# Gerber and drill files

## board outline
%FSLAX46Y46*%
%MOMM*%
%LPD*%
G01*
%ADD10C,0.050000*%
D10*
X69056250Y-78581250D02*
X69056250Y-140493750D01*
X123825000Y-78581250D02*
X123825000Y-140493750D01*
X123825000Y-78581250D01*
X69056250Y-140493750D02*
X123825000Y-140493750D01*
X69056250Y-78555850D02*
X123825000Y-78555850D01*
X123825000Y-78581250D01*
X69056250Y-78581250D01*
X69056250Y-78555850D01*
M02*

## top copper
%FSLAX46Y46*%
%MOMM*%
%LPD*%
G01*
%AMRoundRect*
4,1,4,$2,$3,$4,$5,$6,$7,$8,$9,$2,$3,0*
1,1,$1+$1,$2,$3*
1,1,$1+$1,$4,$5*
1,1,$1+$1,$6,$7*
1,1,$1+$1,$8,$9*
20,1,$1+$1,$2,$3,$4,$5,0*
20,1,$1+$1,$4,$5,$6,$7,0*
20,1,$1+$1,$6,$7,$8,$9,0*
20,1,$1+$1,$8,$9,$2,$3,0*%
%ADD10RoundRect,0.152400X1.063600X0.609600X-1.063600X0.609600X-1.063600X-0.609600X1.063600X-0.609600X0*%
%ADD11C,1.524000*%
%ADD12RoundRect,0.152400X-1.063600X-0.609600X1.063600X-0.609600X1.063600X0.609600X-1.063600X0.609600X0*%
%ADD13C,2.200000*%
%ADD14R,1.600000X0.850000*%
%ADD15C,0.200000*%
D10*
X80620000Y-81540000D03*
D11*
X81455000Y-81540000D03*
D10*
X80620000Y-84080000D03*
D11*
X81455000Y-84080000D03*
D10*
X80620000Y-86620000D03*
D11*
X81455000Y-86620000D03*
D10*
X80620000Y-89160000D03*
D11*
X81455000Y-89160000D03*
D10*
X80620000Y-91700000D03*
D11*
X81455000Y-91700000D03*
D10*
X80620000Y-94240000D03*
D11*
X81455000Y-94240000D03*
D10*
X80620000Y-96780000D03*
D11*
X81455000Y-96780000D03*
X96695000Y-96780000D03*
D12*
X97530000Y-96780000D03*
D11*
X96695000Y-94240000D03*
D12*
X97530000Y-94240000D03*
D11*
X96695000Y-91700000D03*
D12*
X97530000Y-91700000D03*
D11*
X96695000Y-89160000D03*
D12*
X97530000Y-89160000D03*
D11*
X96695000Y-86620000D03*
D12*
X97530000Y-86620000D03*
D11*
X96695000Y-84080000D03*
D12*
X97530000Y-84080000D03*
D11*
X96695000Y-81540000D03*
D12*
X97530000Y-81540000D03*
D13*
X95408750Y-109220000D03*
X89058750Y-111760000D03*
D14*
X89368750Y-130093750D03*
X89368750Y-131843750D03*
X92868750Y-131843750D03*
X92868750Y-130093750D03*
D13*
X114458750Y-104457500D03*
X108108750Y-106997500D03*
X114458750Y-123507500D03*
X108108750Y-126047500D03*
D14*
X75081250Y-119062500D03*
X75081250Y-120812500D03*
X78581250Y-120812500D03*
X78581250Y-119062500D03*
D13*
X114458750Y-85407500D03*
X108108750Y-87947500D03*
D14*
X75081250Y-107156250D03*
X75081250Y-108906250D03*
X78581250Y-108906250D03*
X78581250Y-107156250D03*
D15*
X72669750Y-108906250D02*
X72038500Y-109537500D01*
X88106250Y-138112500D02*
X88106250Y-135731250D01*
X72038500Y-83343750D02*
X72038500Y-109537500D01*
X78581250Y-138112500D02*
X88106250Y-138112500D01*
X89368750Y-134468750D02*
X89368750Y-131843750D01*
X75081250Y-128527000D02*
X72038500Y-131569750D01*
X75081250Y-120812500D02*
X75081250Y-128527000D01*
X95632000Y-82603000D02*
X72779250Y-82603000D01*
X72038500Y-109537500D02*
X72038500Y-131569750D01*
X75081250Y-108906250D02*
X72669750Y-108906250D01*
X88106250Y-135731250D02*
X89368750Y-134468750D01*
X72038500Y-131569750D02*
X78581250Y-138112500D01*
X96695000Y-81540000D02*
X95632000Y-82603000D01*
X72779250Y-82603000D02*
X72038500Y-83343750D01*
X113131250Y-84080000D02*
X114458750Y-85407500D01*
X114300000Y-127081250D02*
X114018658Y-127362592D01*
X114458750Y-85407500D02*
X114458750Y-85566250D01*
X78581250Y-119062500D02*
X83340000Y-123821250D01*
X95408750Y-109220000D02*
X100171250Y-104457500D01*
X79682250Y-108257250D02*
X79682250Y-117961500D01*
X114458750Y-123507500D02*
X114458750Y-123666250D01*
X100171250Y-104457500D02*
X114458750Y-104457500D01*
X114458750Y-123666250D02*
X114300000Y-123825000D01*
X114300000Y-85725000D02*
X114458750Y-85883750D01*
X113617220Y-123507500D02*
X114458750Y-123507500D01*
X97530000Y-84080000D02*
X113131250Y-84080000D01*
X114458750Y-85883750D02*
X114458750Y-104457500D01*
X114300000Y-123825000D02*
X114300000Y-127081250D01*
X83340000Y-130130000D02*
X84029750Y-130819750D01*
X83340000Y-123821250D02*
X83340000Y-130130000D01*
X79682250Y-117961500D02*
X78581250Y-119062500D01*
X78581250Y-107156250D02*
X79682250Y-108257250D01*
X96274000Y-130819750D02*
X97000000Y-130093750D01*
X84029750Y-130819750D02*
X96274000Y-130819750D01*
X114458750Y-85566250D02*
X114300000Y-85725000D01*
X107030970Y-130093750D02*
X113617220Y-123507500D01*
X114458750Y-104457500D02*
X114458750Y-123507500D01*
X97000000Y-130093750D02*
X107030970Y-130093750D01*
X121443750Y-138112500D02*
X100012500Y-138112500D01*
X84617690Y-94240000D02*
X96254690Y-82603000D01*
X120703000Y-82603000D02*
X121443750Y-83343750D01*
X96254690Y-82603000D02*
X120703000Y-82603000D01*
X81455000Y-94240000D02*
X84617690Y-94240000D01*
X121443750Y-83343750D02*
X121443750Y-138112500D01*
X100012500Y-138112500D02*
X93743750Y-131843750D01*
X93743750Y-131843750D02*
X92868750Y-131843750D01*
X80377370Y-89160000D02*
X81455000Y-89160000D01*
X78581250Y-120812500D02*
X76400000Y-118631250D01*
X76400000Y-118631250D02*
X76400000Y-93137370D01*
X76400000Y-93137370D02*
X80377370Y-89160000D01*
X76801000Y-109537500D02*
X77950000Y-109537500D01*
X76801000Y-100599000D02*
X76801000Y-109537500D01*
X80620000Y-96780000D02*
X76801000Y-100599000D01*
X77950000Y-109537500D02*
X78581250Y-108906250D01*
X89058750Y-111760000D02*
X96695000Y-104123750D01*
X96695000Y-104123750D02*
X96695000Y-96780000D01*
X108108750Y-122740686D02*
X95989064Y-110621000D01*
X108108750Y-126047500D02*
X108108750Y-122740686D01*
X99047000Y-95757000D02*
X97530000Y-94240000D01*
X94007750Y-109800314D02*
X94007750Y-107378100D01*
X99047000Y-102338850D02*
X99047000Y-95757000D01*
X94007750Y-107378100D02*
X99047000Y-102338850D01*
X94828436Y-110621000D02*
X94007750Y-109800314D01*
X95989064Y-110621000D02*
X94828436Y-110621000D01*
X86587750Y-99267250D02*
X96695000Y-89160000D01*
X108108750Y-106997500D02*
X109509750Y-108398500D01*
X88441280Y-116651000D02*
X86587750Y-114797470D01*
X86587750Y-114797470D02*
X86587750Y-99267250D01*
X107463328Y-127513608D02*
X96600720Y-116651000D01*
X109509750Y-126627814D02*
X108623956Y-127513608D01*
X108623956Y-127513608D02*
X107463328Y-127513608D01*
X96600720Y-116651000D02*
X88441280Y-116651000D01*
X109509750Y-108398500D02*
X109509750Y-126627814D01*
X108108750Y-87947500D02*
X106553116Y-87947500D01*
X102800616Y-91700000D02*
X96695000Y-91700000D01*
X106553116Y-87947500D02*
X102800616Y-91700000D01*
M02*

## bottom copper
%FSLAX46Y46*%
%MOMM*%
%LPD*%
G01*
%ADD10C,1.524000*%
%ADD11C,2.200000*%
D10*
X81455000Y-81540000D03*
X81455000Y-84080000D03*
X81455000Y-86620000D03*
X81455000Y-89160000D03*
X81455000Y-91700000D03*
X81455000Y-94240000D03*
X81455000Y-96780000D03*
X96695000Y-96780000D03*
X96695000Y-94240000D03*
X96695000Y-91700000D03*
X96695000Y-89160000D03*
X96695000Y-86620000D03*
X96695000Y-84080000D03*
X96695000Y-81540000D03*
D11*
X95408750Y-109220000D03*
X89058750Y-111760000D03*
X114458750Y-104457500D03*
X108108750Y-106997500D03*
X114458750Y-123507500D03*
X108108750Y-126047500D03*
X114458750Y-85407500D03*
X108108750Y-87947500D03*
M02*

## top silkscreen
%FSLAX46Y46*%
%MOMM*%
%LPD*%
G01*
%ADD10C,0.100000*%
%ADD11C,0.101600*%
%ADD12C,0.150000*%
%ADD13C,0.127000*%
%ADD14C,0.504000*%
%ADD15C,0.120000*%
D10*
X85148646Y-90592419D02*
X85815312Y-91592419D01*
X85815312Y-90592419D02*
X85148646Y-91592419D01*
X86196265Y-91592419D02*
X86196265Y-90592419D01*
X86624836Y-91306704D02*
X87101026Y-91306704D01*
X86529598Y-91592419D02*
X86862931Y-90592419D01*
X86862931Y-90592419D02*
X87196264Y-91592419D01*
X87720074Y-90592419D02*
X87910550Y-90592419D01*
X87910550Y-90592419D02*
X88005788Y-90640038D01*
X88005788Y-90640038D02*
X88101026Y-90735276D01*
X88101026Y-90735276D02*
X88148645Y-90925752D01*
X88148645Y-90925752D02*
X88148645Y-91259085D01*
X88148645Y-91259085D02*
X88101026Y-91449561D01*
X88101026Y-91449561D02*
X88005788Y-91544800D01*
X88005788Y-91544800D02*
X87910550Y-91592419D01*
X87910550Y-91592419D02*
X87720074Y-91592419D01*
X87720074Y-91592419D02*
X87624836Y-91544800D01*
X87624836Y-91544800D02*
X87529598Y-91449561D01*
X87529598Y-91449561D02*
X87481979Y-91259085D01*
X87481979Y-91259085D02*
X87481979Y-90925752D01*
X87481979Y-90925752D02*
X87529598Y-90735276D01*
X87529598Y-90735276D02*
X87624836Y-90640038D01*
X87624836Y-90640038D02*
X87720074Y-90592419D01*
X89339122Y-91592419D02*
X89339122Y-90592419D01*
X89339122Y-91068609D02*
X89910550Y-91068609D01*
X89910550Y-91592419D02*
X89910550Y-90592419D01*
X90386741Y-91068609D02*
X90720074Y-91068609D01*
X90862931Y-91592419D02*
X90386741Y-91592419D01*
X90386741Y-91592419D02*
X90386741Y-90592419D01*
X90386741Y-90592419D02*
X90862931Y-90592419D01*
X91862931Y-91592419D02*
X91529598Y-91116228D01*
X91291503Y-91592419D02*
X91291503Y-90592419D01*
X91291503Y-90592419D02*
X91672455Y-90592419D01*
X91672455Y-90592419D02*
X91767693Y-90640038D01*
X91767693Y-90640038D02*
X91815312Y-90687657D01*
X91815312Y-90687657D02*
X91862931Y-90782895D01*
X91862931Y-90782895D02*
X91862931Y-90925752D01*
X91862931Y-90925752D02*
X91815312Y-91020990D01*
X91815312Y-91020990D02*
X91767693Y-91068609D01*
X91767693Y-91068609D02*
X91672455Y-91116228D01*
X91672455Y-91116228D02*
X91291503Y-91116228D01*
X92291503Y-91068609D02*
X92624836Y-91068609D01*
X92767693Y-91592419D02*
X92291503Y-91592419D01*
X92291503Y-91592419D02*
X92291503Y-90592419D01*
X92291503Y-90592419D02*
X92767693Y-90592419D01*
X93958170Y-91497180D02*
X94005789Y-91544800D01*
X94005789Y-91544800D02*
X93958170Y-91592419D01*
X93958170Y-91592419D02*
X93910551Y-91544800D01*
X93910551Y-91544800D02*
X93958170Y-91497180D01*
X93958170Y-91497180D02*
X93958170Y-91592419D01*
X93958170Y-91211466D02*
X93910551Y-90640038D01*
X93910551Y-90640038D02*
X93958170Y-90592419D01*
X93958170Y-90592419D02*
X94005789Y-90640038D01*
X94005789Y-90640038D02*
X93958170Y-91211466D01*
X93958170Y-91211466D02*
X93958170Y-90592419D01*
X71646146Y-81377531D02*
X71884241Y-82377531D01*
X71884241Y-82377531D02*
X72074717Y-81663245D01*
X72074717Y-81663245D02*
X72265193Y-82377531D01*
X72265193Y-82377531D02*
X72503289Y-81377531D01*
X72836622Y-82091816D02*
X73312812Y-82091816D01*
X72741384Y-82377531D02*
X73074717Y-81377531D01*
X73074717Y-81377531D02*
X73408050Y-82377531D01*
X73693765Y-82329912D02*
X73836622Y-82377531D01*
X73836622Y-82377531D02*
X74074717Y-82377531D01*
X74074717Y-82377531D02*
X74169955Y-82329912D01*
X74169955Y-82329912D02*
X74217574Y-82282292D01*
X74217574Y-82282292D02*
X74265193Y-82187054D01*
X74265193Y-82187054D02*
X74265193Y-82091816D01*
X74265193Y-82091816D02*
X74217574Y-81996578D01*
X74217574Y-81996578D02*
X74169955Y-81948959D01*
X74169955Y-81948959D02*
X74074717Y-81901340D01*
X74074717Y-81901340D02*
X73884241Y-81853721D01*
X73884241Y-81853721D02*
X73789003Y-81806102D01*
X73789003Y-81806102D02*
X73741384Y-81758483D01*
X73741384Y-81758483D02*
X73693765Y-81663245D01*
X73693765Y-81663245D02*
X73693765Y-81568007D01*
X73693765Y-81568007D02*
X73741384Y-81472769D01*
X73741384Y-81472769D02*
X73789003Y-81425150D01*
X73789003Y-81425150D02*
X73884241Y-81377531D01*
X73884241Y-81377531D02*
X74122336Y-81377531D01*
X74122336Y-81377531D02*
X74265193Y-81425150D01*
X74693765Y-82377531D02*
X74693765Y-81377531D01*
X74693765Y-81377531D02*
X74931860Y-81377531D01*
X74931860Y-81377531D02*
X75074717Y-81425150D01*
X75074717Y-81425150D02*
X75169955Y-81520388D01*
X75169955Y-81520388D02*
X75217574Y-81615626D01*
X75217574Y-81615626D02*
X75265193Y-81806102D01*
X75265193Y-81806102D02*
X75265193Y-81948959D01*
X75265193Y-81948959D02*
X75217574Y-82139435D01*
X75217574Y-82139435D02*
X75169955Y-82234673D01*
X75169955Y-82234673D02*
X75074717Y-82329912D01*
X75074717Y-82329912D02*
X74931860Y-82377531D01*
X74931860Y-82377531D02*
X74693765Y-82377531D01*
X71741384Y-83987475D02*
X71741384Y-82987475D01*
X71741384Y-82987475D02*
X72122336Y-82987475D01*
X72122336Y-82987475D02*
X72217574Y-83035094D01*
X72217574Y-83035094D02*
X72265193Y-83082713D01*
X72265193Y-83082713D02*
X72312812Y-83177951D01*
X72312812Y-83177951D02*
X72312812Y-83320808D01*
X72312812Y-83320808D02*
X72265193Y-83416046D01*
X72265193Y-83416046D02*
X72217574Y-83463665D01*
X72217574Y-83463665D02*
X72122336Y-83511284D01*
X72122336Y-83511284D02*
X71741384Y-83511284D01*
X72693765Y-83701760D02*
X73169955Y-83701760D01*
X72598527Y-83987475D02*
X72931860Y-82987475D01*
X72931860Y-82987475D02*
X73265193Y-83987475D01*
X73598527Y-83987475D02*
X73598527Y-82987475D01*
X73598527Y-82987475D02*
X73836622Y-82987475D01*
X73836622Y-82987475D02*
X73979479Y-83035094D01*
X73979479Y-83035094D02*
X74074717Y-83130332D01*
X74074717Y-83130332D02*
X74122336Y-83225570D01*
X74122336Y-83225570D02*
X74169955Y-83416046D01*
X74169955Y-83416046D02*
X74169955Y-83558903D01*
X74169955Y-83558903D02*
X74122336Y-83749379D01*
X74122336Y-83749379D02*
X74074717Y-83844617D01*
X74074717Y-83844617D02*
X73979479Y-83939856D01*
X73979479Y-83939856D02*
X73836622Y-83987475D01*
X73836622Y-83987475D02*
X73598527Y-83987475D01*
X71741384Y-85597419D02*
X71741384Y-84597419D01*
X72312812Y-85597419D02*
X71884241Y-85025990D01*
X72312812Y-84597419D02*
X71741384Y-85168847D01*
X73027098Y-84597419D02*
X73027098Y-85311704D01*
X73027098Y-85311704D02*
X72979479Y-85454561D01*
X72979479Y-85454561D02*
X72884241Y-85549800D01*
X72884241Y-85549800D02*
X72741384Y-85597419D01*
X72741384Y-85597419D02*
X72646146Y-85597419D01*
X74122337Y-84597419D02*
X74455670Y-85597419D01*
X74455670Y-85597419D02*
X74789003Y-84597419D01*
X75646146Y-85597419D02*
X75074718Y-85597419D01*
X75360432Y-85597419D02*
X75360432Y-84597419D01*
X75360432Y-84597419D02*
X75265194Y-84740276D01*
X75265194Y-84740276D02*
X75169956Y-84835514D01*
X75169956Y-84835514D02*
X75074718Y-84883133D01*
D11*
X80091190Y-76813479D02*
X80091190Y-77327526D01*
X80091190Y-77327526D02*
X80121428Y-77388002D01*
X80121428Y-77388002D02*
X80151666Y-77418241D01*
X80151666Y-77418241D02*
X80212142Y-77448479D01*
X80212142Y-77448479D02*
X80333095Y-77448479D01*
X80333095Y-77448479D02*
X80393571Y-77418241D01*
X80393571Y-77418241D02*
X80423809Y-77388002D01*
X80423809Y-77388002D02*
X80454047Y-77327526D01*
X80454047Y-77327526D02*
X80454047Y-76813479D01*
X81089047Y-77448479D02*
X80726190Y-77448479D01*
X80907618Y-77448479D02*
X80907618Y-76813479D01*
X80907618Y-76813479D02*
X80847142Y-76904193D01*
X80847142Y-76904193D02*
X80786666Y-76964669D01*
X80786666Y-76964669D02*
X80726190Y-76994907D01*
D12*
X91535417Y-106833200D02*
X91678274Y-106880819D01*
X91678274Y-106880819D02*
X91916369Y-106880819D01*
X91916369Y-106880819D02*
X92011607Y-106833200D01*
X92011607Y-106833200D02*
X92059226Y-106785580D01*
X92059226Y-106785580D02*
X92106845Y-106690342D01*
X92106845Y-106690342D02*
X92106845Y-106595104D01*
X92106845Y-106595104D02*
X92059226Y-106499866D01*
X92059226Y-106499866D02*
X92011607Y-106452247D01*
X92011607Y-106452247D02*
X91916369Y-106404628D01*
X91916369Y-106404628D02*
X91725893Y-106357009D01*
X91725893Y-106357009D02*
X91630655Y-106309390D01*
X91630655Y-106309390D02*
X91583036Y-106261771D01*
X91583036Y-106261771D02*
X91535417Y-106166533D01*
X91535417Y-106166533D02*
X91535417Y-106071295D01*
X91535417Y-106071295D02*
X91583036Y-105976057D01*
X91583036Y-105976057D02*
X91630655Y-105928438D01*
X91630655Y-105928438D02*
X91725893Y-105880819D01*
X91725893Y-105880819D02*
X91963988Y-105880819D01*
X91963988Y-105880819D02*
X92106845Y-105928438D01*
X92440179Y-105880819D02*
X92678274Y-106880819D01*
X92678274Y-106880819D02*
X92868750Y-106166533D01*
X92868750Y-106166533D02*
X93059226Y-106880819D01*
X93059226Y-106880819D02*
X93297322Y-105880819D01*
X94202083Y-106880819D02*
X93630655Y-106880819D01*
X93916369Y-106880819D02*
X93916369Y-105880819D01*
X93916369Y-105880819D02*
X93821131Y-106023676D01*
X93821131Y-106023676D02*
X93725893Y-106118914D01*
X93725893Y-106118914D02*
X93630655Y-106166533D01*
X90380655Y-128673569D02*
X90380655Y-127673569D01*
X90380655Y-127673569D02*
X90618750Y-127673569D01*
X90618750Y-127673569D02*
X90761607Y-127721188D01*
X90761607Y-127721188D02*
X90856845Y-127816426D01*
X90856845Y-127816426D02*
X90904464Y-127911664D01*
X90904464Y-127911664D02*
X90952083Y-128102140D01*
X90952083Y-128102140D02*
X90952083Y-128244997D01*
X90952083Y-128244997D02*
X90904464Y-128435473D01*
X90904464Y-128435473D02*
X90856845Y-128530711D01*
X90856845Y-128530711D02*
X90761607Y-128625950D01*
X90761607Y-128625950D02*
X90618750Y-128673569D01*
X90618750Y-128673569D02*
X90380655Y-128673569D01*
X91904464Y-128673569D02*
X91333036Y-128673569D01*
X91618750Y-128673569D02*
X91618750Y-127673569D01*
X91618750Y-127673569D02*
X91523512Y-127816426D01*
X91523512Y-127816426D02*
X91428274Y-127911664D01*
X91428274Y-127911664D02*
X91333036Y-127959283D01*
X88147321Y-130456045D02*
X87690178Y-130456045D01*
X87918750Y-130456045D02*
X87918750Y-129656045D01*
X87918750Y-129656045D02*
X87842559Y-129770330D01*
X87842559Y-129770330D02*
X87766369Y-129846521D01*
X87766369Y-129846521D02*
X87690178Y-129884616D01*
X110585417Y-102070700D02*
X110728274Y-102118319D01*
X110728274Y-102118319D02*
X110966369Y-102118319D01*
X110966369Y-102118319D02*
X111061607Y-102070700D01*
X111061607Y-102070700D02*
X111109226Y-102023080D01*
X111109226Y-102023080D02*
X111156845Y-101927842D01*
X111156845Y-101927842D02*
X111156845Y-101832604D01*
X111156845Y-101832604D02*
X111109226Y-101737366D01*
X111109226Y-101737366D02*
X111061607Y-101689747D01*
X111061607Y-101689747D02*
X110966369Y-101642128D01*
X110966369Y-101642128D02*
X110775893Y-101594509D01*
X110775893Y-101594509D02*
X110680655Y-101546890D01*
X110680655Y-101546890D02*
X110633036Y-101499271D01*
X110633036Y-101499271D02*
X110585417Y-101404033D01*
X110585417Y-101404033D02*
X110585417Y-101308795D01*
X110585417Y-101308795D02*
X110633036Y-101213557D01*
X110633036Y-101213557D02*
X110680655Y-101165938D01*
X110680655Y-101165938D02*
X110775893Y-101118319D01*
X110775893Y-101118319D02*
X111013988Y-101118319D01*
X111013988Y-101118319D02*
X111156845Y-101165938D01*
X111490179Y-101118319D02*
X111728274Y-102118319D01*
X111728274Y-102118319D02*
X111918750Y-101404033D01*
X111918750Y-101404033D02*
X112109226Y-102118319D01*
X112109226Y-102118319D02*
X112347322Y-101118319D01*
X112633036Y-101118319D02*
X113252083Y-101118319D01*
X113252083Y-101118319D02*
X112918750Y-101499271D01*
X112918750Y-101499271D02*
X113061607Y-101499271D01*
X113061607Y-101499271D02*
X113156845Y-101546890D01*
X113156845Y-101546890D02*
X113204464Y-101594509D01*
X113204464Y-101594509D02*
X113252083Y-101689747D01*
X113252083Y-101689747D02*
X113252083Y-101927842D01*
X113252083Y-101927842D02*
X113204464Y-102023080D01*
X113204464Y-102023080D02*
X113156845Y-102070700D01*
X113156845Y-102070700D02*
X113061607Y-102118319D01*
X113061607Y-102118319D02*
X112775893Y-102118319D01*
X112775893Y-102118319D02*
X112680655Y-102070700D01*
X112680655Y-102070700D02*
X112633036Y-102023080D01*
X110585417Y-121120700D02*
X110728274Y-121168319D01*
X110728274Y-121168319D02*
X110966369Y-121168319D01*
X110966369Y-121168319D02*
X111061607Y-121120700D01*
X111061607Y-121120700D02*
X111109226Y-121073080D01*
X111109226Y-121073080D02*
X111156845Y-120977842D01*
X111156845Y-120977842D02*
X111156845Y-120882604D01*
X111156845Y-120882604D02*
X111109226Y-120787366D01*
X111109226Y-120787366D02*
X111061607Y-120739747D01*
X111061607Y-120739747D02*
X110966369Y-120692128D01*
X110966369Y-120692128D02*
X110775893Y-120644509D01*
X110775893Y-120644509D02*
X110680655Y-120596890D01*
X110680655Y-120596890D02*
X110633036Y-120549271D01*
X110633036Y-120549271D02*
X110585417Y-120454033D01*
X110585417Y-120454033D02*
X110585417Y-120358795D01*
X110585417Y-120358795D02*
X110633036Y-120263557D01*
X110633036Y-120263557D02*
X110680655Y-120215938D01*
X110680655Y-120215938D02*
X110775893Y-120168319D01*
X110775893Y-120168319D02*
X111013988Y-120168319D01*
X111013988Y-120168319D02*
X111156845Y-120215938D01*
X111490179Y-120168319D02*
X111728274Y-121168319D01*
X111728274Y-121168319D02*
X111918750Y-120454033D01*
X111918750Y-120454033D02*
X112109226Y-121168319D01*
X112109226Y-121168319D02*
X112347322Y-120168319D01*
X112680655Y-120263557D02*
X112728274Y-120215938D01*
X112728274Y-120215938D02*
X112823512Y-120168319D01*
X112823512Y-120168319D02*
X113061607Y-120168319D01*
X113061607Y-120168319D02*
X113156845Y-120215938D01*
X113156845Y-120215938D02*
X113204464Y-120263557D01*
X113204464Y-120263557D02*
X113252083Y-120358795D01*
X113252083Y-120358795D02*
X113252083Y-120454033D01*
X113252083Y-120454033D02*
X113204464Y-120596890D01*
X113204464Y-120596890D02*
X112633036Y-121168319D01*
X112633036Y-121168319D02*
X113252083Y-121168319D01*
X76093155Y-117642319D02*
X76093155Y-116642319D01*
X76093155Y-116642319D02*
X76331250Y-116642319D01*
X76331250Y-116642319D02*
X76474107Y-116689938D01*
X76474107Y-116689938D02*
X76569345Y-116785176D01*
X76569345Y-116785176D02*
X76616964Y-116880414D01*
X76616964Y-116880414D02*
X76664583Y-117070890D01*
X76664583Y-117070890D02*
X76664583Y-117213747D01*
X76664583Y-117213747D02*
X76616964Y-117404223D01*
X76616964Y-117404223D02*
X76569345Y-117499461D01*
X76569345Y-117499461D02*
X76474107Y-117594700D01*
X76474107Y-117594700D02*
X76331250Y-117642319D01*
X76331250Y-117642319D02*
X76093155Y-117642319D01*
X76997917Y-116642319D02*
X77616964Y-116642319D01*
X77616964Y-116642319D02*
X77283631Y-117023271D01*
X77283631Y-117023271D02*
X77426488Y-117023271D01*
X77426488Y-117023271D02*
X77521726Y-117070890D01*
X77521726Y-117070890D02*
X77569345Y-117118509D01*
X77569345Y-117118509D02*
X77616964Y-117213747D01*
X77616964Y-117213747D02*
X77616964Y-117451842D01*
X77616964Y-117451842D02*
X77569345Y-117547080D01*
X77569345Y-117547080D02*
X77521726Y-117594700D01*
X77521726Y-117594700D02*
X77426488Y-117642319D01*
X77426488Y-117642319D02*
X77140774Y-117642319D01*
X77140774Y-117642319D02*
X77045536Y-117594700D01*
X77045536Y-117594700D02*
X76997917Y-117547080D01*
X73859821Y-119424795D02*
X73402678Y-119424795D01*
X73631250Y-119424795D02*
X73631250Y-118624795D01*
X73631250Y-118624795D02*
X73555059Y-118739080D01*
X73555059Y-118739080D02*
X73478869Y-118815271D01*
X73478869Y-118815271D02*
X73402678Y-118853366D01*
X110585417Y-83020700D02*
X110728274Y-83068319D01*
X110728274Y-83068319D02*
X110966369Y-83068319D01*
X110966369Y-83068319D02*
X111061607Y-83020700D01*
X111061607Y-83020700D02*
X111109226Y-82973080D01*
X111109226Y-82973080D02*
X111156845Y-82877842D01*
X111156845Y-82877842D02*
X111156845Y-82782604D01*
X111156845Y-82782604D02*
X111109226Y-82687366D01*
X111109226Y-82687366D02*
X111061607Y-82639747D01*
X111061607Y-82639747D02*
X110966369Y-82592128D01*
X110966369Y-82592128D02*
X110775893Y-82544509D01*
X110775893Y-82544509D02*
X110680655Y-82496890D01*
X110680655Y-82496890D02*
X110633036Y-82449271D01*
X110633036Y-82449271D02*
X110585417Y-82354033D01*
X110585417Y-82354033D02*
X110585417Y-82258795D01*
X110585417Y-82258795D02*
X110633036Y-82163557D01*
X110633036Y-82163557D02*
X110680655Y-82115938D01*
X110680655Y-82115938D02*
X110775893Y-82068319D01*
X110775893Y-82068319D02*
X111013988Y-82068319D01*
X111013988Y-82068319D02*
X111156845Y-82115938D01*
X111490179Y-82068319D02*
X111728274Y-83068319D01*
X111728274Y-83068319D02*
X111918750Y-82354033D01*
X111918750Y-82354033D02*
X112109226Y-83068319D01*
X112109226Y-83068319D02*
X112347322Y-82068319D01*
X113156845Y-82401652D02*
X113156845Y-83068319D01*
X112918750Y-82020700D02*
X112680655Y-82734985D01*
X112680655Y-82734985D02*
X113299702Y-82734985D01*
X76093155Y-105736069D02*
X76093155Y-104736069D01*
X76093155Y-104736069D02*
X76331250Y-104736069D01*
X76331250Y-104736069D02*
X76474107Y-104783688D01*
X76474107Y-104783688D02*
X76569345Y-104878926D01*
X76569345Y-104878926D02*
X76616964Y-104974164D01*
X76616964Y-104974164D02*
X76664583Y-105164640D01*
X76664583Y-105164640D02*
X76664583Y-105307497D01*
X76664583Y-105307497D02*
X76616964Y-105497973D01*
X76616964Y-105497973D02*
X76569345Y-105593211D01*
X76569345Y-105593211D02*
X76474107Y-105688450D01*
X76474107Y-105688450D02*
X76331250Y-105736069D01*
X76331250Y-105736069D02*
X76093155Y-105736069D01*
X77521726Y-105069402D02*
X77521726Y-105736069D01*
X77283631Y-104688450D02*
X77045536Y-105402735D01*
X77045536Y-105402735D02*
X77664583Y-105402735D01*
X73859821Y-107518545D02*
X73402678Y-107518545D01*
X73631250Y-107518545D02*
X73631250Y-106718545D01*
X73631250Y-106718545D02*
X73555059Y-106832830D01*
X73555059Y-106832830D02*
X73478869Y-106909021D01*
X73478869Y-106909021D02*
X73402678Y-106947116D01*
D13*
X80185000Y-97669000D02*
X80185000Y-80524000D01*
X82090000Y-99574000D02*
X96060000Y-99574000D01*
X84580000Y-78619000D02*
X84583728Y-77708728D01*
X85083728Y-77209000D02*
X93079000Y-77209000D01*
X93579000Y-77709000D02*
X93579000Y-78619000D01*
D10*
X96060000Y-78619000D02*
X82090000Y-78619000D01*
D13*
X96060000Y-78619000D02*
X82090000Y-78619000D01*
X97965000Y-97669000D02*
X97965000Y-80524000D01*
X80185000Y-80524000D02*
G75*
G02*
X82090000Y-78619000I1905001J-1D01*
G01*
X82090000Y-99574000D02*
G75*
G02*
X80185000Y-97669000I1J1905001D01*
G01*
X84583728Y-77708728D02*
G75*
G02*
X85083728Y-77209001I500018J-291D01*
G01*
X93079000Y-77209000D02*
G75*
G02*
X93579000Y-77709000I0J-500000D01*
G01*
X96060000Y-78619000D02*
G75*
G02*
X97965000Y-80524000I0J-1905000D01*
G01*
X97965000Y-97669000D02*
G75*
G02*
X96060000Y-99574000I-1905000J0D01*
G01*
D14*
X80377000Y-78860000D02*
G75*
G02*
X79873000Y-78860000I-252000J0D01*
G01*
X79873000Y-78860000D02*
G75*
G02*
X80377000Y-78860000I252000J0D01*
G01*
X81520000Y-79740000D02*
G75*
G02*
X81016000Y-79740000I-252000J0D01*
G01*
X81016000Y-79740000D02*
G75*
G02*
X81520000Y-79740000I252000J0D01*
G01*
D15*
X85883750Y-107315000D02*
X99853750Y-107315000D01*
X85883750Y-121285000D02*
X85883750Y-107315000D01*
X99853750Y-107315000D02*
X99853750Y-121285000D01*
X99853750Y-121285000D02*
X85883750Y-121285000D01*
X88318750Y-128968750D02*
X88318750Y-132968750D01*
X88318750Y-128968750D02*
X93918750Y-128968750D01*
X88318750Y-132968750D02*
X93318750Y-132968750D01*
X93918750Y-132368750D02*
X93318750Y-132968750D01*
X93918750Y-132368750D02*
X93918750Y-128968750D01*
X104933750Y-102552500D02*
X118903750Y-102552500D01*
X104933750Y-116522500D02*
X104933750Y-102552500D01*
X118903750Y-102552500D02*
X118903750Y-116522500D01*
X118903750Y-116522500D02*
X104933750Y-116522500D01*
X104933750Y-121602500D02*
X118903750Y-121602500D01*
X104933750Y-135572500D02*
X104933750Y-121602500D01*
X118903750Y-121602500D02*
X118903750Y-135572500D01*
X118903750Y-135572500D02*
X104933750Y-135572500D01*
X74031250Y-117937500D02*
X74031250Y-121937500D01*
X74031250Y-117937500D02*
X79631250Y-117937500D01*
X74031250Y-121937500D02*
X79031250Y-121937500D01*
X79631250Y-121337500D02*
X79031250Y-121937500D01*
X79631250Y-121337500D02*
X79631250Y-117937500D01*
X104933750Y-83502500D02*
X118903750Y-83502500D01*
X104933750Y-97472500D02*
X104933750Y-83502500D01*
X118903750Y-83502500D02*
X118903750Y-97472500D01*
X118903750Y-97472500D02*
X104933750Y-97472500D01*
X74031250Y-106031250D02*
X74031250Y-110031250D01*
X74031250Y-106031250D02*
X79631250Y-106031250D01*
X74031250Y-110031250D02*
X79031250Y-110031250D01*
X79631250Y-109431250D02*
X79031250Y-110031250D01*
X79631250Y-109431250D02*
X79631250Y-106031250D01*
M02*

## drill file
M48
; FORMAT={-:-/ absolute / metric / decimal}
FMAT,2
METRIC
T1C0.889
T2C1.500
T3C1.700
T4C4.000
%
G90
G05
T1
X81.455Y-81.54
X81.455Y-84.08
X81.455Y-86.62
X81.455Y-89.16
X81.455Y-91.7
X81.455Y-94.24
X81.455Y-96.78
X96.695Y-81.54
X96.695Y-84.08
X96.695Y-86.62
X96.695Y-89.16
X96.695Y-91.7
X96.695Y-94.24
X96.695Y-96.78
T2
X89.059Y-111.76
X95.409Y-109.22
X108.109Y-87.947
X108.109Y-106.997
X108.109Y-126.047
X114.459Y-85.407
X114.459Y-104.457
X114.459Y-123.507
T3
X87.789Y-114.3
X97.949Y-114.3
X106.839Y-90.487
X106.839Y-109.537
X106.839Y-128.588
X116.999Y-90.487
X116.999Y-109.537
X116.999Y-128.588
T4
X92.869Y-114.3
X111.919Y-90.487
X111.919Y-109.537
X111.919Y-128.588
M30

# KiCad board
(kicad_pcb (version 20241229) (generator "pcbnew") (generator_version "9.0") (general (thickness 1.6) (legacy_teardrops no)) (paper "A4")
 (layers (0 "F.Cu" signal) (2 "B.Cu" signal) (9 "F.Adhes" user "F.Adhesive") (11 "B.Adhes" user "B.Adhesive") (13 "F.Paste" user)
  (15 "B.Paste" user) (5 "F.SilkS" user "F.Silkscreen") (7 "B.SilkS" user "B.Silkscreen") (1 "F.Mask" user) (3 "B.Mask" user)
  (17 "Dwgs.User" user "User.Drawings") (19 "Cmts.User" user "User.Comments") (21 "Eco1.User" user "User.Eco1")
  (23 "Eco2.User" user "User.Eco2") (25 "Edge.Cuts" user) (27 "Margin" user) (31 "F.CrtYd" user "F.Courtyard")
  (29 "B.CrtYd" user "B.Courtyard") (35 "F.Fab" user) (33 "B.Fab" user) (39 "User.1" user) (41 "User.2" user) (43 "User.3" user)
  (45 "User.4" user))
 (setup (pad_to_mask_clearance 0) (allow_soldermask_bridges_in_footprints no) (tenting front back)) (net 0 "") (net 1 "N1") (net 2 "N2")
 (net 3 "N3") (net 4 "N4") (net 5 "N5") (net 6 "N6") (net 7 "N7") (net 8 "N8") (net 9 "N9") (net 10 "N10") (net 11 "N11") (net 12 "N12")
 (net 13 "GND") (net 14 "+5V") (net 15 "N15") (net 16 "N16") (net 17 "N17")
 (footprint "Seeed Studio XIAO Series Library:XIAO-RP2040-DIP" (layer "F.Cu") (at 89.075 89.16)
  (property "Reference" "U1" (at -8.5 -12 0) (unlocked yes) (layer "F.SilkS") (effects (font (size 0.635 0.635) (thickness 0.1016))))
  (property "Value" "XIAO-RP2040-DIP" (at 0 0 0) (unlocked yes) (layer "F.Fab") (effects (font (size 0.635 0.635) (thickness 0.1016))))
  (fp_line (start -8.89 8.509) (end -8.89 -8.636) (stroke (width 0.127) (type solid)) (layer "F.SilkS"))
  (fp_line (start -6.985 10.414) (end 6.985 10.414) (stroke (width 0.127) (type solid)) (layer "F.SilkS"))
  (fp_line (start -4.495 -10.541) (end -4.491272 -11.451272) (stroke (width 0.127) (type solid)) (layer "F.SilkS"))
  (fp_line (start -3.991272 -11.951) (end 4.004 -11.951) (stroke (width 0.127) (type solid)) (layer "F.SilkS"))
  (fp_line (start 4.504 -11.451) (end 4.504 -10.541) (stroke (width 0.127) (type solid)) (layer "F.SilkS"))
  (fp_line (start 6.985 -10.541) (end -6.985 -10.541) (stroke (width 0.1) (type solid)) (layer "F.SilkS"))
  (fp_line (start 6.985 -10.541) (end -6.985 -10.541) (stroke (width 0.127) (type solid)) (layer "F.SilkS"))
  (fp_line (start 8.89 8.509) (end 8.89 -8.636) (stroke (width 0.127) (type solid)) (layer "F.SilkS"))
  (fp_arc (start -8.89 -8.636) (mid -8.332038 -9.983038) (end -6.985 -10.541) (stroke (width 0.127) (type solid)) (layer "F.SilkS"))
  (fp_arc (start -6.985 10.414) (mid -8.332038 9.856038) (end -8.89 8.509) (stroke (width 0.127) (type solid)) (layer "F.SilkS"))
  (fp_arc (start -4.491272 -11.451272) (mid -4.344728 -11.80464) (end -3.991272 -11.951) (stroke (width 0.127) (type default))
   (layer "F.SilkS"))
  (fp_arc (start 4.004 -11.951) (mid 4.357553 -11.804553) (end 4.504 -11.451) (stroke (width 0.127) (type default)) (layer "F.SilkS"))
  (fp_arc (start 6.985 -10.541) (mid 8.332038 -9.983038) (end 8.89 -8.636) (stroke (width 0.127) (type solid)) (layer "F.SilkS"))
  (fp_arc (start 8.89 8.509) (mid 8.332038 9.856038) (end 6.985 10.414) (stroke (width 0.127) (type solid)) (layer "F.SilkS"))
  (fp_circle (center -8.95 -10.3) (end -8.95 -10.554) (stroke (width 0.5) (type solid)) (fill yes) (layer "F.SilkS"))
  (fp_circle (center -7.807 -9.42) (end -7.807 -9.674) (stroke (width 0.5) (type solid)) (fill yes) (layer "F.SilkS"))
  (pad "1" smd roundrect (at -8.455 -7.62 180) (size 2.432 1.524) (layers "F.Cu" "F.Mask") (roundrect_rratio 0.1) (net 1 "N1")
   (thermal_bridge_angle 45))
  (pad "1" thru_hole circle (at -7.62 -7.62 180) (size 1.524 1.524) (drill 0.889) (layers "*.Cu" "*.Mask") (remove_unused_layers no)
   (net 1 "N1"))
  (pad "2" smd roundrect (at -8.455 -5.08 180) (size 2.432 1.524) (layers "F.Cu" "F.Mask") (roundrect_rratio 0.1) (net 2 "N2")
   (thermal_bridge_angle 45))
  (pad "2" thru_hole circle (at -7.62 -5.08 180) (size 1.524 1.524) (drill 0.889) (layers "*.Cu" "*.Mask") (remove_unused_layers no)
   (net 2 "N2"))
  (pad "3" smd roundrect (at -8.455 -2.54 180) (size 2.432 1.524) (layers "F.Cu" "F.Mask") (roundrect_rratio 0.1) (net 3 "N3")
   (thermal_bridge_angle 45))
  (pad "3" thru_hole circle (at -7.62 -2.54 180) (size 1.524 1.524) (drill 0.889) (layers "*.Cu" "*.Mask") (remove_unused_layers no)
   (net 3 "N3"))
  (pad "4" smd roundrect (at -8.455 0 180) (size 2.432 1.524) (layers "F.Cu" "F.Mask") (roundrect_rratio 0.1) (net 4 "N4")
   (thermal_bridge_angle 45))
  (pad "4" thru_hole circle (at -7.62 0 180) (size 1.524 1.524) (drill 0.889) (layers "*.Cu" "*.Mask") (remove_unused_layers no)
   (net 4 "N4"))
  (pad "5" smd roundrect (at -8.455 2.54 180) (size 2.432 1.524) (layers "F.Cu" "F.Mask") (roundrect_rratio 0.1) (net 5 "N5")
   (thermal_bridge_angle 45))
  (pad "5" thru_hole circle (at -7.62 2.54 180) (size 1.524 1.524) (drill 0.889) (layers "*.Cu" "*.Mask") (remove_unused_layers no)
   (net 5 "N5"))
  (pad "6" smd roundrect (at -8.455 5.08 180) (size 2.432 1.524) (layers "F.Cu" "F.Mask") (roundrect_rratio 0.1) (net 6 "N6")
   (thermal_bridge_angle 45))
  (pad "6" thru_hole circle (at -7.62 5.08 180) (size 1.524 1.524) (drill 0.889) (layers "*.Cu" "*.Mask") (remove_unused_layers no)
   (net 6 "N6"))
  (pad "7" smd roundrect (at -8.455 7.62 180) (size 2.432 1.524) (layers "F.Cu" "F.Mask") (roundrect_rratio 0.1) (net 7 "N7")
   (thermal_bridge_angle 45))
  (pad "7" thru_hole circle (at -7.62 7.62 180) (size 1.524 1.524) (drill 0.889) (layers "*.Cu" "*.Mask") (remove_unused_layers no)
   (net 7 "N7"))
  (pad "8" thru_hole circle (at 7.62 7.62) (size 1.524 1.524) (drill 0.889) (layers "*.Cu" "*.Mask") (remove_unused_layers no) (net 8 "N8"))
  (pad "8" smd roundrect (at 8.455 7.62) (size 2.432 1.524) (layers "F.Cu" "F.Mask") (roundrect_rratio 0.1) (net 8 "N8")
   (thermal_bridge_angle 45))
  (pad "9" thru_hole circle (at 7.62 5.08) (size 1.524 1.524) (drill 0.889) (layers "*.Cu" "*.Mask") (remove_unused_layers no) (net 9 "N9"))
  (pad "9" smd roundrect (at 8.455 5.08) (size 2.432 1.524) (layers "F.Cu" "F.Mask") (roundrect_rratio 0.1) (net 9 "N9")
   (thermal_bridge_angle 45))
  (pad "10" thru_hole circle (at 7.62 2.54) (size 1.524 1.524) (drill 0.889) (layers "*.Cu" "*.Mask") (remove_unused_layers no)
   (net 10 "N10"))
  (pad "10" smd roundrect (at 8.455 2.54) (size 2.432 1.524) (layers "F.Cu" "F.Mask") (roundrect_rratio 0.1) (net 10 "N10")
   (thermal_bridge_angle 45))
  (pad "11" thru_hole circle (at 7.62 0) (size 1.524 1.524) (drill 0.889) (layers "*.Cu" "*.Mask") (remove_unused_layers no) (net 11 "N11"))
  (pad "11" smd roundrect (at 8.455 0) (size 2.432 1.524) (layers "F.Cu" "F.Mask") (roundrect_rratio 0.1) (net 11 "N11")
   (thermal_bridge_angle 45))
  (pad "12" thru_hole circle (at 7.62 -2.54) (size 1.524 1.524) (drill 0.889) (layers "*.Cu" "*.Mask") (remove_unused_layers no)
   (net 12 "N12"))
  (pad "12" smd roundrect (at 8.455 -2.54) (size 2.432 1.524) (layers "F.Cu" "F.Mask") (roundrect_rratio 0.1) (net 12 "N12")
   (thermal_bridge_angle 45))
  (pad "13" thru_hole circle (at 7.62 -5.08) (size 1.524 1.524) (drill 0.889) (layers "*.Cu" "*.Mask") (remove_unused_layers no)
   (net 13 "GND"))
  (pad "13" smd roundrect (at 8.455 -5.08) (size 2.432 1.524) (layers "F.Cu" "F.Mask") (roundrect_rratio 0.1) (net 13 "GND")
   (thermal_bridge_angle 45))
  (pad "14" thru_hole circle (at 7.62 -7.62) (size 1.524 1.524) (drill 0.889) (layers "*.Cu" "*.Mask") (remove_unused_layers no)
   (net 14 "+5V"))
  (pad "14" smd roundrect (at 8.455 -7.62) (size 2.432 1.524) (layers "F.Cu" "F.Mask") (roundrect_rratio 0.1) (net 14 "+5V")
   (thermal_bridge_angle 45)))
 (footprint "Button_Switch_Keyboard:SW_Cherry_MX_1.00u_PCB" (layer "F.Cu") (at 95.40875 109.22)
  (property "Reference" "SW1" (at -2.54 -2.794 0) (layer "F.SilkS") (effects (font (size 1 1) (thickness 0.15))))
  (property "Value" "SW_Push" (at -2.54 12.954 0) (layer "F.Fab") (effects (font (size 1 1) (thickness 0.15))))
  (fp_line (start -9.525 -1.905) (end 4.445 -1.905) (stroke (width 0.12) (type solid)) (layer "F.SilkS"))
  (fp_line (start -9.525 12.065) (end -9.525 -1.905) (stroke (width 0.12) (type solid)) (layer "F.SilkS"))
  (fp_line (start 4.445 -1.905) (end 4.445 12.065) (stroke (width 0.12) (type solid)) (layer "F.SilkS"))
  (fp_line (start 4.445 12.065) (end -9.525 12.065) (stroke (width 0.12) (type solid)) (layer "F.SilkS"))
  (pad "" np_thru_hole circle (at -7.62 5.08) (size 1.7 1.7) (drill 1.7) (layers "*.Cu" "*.Mask"))
  (pad "" np_thru_hole circle (at -2.54 5.08) (size 4 4) (drill 4) (layers "*.Cu" "*.Mask"))
  (pad "" np_thru_hole circle (at 2.54 5.08) (size 1.7 1.7) (drill 1.7) (layers "*.Cu" "*.Mask"))
  (pad "1" thru_hole circle (at 0 0) (size 2.2 2.2) (drill 1.5) (layers "*.Cu" "*.Mask") (remove_unused_layers no) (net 13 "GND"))
  (pad "2" thru_hole circle (at -6.35 2.54) (size 2.2 2.2) (drill 1.5) (layers "*.Cu" "*.Mask") (remove_unused_layers no) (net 8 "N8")))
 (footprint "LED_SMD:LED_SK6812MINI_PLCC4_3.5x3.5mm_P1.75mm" (layer "F.Cu") (at 91.11875 130.96875)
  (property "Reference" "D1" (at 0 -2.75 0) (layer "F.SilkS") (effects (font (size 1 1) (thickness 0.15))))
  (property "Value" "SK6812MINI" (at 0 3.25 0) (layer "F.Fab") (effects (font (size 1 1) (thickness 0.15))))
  (fp_line (start -2.8 -2) (end -2.8 2) (stroke (width 0.12) (type default)) (layer "F.SilkS"))
  (fp_line (start -2.8 -2) (end 2.8 -2) (stroke (width 0.12) (type solid)) (layer "F.SilkS"))
  (fp_line (start -2.8 2) (end 2.2 2) (stroke (width 0.12) (type solid)) (layer "F.SilkS"))
  (fp_line (start 2.8 1.4) (end 2.2 2) (stroke (width 0.12) (type default)) (layer "F.SilkS"))
  (fp_line (start 2.8 1.4) (end 2.8 -2) (stroke (width 0.12) (type solid)) (layer "F.SilkS"))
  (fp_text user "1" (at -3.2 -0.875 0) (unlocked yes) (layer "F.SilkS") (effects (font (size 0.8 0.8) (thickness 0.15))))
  (pad "1" smd rect (at -1.75 -0.875) (size 1.6 0.85) (layers "F.Cu" "F.Mask" "F.Paste") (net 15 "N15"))
  (pad "2" smd rect (at -1.75 0.875) (size 1.6 0.85) (layers "F.Cu" "F.Mask" "F.Paste") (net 14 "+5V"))
  (pad "3" smd rect (at 1.75 0.875) (size 1.6 0.85) (layers "F.Cu" "F.Mask" "F.Paste") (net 6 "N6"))
  (pad "4" smd rect (at 1.75 -0.875) (size 1.6 0.85) (layers "F.Cu" "F.Mask" "F.Paste") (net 13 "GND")))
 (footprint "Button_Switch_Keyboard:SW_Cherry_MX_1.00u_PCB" (layer "F.Cu") (at 114.45875 104.4575)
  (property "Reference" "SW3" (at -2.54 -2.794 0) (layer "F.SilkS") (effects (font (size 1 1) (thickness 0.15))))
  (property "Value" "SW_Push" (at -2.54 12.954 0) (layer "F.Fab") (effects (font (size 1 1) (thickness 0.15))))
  (fp_line (start -9.525 -1.905) (end 4.445 -1.905) (stroke (width 0.12) (type solid)) (layer "F.SilkS"))
  (fp_line (start -9.525 12.065) (end -9.525 -1.905) (stroke (width 0.12) (type solid)) (layer "F.SilkS"))
  (fp_line (start 4.445 -1.905) (end 4.445 12.065) (stroke (width 0.12) (type solid)) (layer "F.SilkS"))
  (fp_line (start 4.445 12.065) (end -9.525 12.065) (stroke (width 0.12) (type solid)) (layer "F.SilkS"))
  (pad "" np_thru_hole circle (at -7.62 5.08) (size 1.7 1.7) (drill 1.7) (layers "*.Cu" "*.Mask"))
  (pad "" np_thru_hole circle (at -2.54 5.08) (size 4 4) (drill 4) (layers "*.Cu" "*.Mask"))
  (pad "" np_thru_hole circle (at 2.54 5.08) (size 1.7 1.7) (drill 1.7) (layers "*.Cu" "*.Mask"))
  (pad "1" thru_hole circle (at 0 0) (size 2.2 2.2) (drill 1.5) (layers "*.Cu" "*.Mask") (remove_unused_layers no) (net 13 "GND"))
  (pad "2" thru_hole circle (at -6.35 2.54) (size 2.2 2.2) (drill 1.5) (layers "*.Cu" "*.Mask") (remove_unused_layers no) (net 11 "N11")))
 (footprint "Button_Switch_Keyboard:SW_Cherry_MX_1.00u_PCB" (layer "F.Cu") (at 114.45875 123.5075)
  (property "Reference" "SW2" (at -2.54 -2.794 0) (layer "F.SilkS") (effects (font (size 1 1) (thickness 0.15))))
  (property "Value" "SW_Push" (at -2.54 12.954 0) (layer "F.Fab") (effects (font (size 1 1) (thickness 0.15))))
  (fp_line (start -9.525 -1.905) (end 4.445 -1.905) (stroke (width 0.12) (type solid)) (layer "F.SilkS"))
  (fp_line (start -9.525 12.065) (end -9.525 -1.905) (stroke (width 0.12) (type solid)) (layer "F.SilkS"))
  (fp_line (start 4.445 -1.905) (end 4.445 12.065) (stroke (width 0.12) (type solid)) (layer "F.SilkS"))
  (fp_line (start 4.445 12.065) (end -9.525 12.065) (stroke (width 0.12) (type solid)) (layer "F.SilkS"))
  (pad "" np_thru_hole circle (at -7.62 5.08) (size 1.7 1.7) (drill 1.7) (layers "*.Cu" "*.Mask"))
  (pad "" np_thru_hole circle (at -2.54 5.08) (size 4 4) (drill 4) (layers "*.Cu" "*.Mask"))
  (pad "" np_thru_hole circle (at 2.54 5.08) (size 1.7 1.7) (drill 1.7) (layers "*.Cu" "*.Mask"))
  (pad "1" thru_hole circle (at 0 0) (size 2.2 2.2) (drill 1.5) (layers "*.Cu" "*.Mask") (remove_unused_layers no) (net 13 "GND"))
  (pad "2" thru_hole circle (at -6.35 2.54) (size 2.2 2.2) (drill 1.5) (layers "*.Cu" "*.Mask") (remove_unused_layers no) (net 9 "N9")))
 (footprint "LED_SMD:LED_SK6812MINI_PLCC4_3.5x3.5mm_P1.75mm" (layer "F.Cu") (at 76.83125 119.9375)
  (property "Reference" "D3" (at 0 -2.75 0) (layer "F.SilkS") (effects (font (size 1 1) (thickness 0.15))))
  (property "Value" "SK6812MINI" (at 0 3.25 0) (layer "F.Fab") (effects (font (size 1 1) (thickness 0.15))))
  (fp_line (start -2.8 -2) (end -2.8 2) (stroke (width 0.12) (type default)) (layer "F.SilkS"))
  (fp_line (start -2.8 -2) (end 2.8 -2) (stroke (width 0.12) (type solid)) (layer "F.SilkS"))
  (fp_line (start -2.8 2) (end 2.2 2) (stroke (width 0.12) (type solid)) (layer "F.SilkS"))
  (fp_line (start 2.8 1.4) (end 2.2 2) (stroke (width 0.12) (type default)) (layer "F.SilkS"))
  (fp_line (start 2.8 1.4) (end 2.8 -2) (stroke (width 0.12) (type solid)) (layer "F.SilkS"))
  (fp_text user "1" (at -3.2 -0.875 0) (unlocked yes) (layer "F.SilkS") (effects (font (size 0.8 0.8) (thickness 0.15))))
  (pad "1" smd rect (at -1.75 -0.875) (size 1.6 0.85) (layers "F.Cu" "F.Mask" "F.Paste") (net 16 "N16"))
  (pad "2" smd rect (at -1.75 0.875) (size 1.6 0.85) (layers "F.Cu" "F.Mask" "F.Paste") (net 14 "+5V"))
  (pad "3" smd rect (at 1.75 0.875) (size 1.6 0.85) (layers "F.Cu" "F.Mask" "F.Paste") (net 4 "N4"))
  (pad "4" smd rect (at 1.75 -0.875) (size 1.6 0.85) (layers "F.Cu" "F.Mask" "F.Paste") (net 13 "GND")))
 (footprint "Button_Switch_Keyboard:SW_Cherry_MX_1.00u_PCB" (layer "F.Cu") (at 114.45875 85.4075)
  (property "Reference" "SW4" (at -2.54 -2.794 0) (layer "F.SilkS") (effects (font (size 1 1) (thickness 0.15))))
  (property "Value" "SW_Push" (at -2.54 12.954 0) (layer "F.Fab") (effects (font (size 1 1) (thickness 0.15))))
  (fp_line (start -9.525 -1.905) (end 4.445 -1.905) (stroke (width 0.12) (type solid)) (layer "F.SilkS"))
  (fp_line (start -9.525 12.065) (end -9.525 -1.905) (stroke (width 0.12) (type solid)) (layer "F.SilkS"))
  (fp_line (start 4.445 -1.905) (end 4.445 12.065) (stroke (width 0.12) (type solid)) (layer "F.SilkS"))
  (fp_line (start 4.445 12.065) (end -9.525 12.065) (stroke (width 0.12) (type solid)) (layer "F.SilkS"))
  (pad "" np_thru_hole circle (at -7.62 5.08) (size 1.7 1.7) (drill 1.7) (layers "*.Cu" "*.Mask"))
  (pad "" np_thru_hole circle (at -2.54 5.08) (size 4 4) (drill 4) (layers "*.Cu" "*.Mask"))
  (pad "" np_thru_hole circle (at 2.54 5.08) (size 1.7 1.7) (drill 1.7) (layers "*.Cu" "*.Mask"))
  (pad "1" thru_hole circle (at 0 0) (size 2.2 2.2) (drill 1.5) (layers "*.Cu" "*.Mask") (remove_unused_layers no) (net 13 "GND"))
  (pad "2" thru_hole circle (at -6.35 2.54) (size 2.2 2.2) (drill 1.5) (layers "*.Cu" "*.Mask") (remove_unused_layers no) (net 10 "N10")))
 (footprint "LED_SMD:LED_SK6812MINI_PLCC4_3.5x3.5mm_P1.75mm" (layer "F.Cu") (at 76.83125 108.03125)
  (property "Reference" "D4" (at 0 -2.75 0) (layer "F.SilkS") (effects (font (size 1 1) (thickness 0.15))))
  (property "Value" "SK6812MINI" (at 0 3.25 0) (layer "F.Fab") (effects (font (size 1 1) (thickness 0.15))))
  (fp_line (start -2.8 -2) (end -2.8 2) (stroke (width 0.12) (type default)) (layer "F.SilkS"))
  (fp_line (start -2.8 -2) (end 2.8 -2) (stroke (width 0.12) (type solid)) (layer "F.SilkS"))
  (fp_line (start -2.8 2) (end 2.2 2) (stroke (width 0.12) (type solid)) (layer "F.SilkS"))
  (fp_line (start 2.8 1.4) (end 2.2 2) (stroke (width 0.12) (type default)) (layer "F.SilkS"))
  (fp_line (start 2.8 1.4) (end 2.8 -2) (stroke (width 0.12) (type solid)) (layer "F.SilkS"))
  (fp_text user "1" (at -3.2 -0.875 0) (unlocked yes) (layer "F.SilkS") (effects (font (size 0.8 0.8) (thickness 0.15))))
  (pad "1" smd rect (at -1.75 -0.875) (size 1.6 0.85) (layers "F.Cu" "F.Mask" "F.Paste") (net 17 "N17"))
  (pad "2" smd rect (at -1.75 0.875) (size 1.6 0.85) (layers "F.Cu" "F.Mask" "F.Paste") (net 14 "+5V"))
  (pad "3" smd rect (at 1.75 0.875) (size 1.6 0.85) (layers "F.Cu" "F.Mask" "F.Paste") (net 7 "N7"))
  (pad "4" smd rect (at 1.75 -0.875) (size 1.6 0.85) (layers "F.Cu" "F.Mask" "F.Paste") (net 13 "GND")))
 (gr_line (start 69.05625 78.58125) (end 69.05625 140.49375) (stroke (width 0.05) (type default)) (layer "Edge.Cuts"))
 (gr_rect (start 123.825 78.58125) (end 123.825 140.49375) (stroke (width 0.05) (type default)) (fill no) (layer "Edge.Cuts"))
 (gr_line (start 69.05625 140.49375) (end 123.825 140.49375) (stroke (width 0.05) (type default)) (layer "Edge.Cuts"))
 (gr_rect (start 69.05625 78.55585) (end 123.825 78.58125) (stroke (width 0.05) (type default)) (fill no) (layer "Edge.Cuts"))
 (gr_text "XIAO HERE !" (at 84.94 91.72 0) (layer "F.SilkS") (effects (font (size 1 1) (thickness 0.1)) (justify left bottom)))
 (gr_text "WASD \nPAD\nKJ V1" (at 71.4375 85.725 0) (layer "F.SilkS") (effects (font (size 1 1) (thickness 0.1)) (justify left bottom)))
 (segment (start 72.66975 108.90625) (end 72.0385 109.5375) (width 0.2) (layer "F.Cu") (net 14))
 (segment (start 88.10625 138.1125) (end 88.10625 135.73125) (width 0.2) (layer "F.Cu") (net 14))
 (segment (start 72.0385 83.34375) (end 72.0385 109.5375) (width 0.2) (layer "F.Cu") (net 14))
 (segment (start 78.58125 138.1125) (end 88.10625 138.1125) (width 0.2) (layer "F.Cu") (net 14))
 (segment (start 89.36875 134.46875) (end 89.36875 131.84375) (width 0.2) (layer "F.Cu") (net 14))
 (segment (start 75.08125 128.527) (end 72.0385 131.56975) (width 0.2) (layer "F.Cu") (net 14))
 (segment (start 75.08125 120.8125) (end 75.08125 128.527) (width 0.2) (layer "F.Cu") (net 14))
 (segment (start 95.632 82.603) (end 72.77925 82.603) (width 0.2) (layer "F.Cu") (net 14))
 (segment (start 72.0385 109.5375) (end 72.0385 131.56975) (width 0.2) (layer "F.Cu") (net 14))
 (segment (start 75.08125 108.90625) (end 72.66975 108.90625) (width 0.2) (layer "F.Cu") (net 14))
 (segment (start 88.10625 135.73125) (end 89.36875 134.46875) (width 0.2) (layer "F.Cu") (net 14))
 (segment (start 72.0385 131.56975) (end 78.58125 138.1125) (width 0.2) (layer "F.Cu") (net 14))
 (segment (start 96.695 81.54) (end 95.632 82.603) (width 0.2) (layer "F.Cu") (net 14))
 (segment (start 72.77925 82.603) (end 72.0385 83.34375) (width 0.2) (layer "F.Cu") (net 14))
 (segment (start 113.13125 84.08) (end 114.45875 85.4075) (width 0.2) (layer "F.Cu") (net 13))
 (segment (start 114.3 127.08125) (end 114.018658 127.362592) (width 0.2) (layer "F.Cu") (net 13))
 (segment (start 114.45875 85.4075) (end 114.45875 85.56625) (width 0.2) (layer "F.Cu") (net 13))
 (segment (start 78.58125 119.0625) (end 83.34 123.82125) (width 0.2) (layer "F.Cu") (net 13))
 (segment (start 95.40875 109.22) (end 100.17125 104.4575) (width 0.2) (layer "F.Cu") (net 13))
 (segment (start 79.68225 108.25725) (end 79.68225 117.9615) (width 0.2) (layer "F.Cu") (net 13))
 (segment (start 114.45875 123.5075) (end 114.45875 123.66625) (width 0.2) (layer "F.Cu") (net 13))
 (segment (start 100.17125 104.4575) (end 114.45875 104.4575) (width 0.2) (layer "F.Cu") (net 13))
 (segment (start 114.45875 123.66625) (end 114.3 123.825) (width 0.2) (layer "F.Cu") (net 13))
 (segment (start 114.3 85.725) (end 114.45875 85.88375) (width 0.2) (layer "F.Cu") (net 13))
 (segment (start 113.61722 123.5075) (end 114.45875 123.5075) (width 0.2) (layer "F.Cu") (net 13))
 (segment (start 97.53 84.08) (end 113.13125 84.08) (width 0.2) (layer "F.Cu") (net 13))
 (segment (start 114.45875 85.88375) (end 114.45875 104.4575) (width 0.2) (layer "F.Cu") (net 13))
 (segment (start 114.3 123.825) (end 114.3 127.08125) (width 0.2) (layer "F.Cu") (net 13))
 (segment (start 83.34 130.13) (end 84.02975 130.81975) (width 0.2) (layer "F.Cu") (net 13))
 (segment (start 83.34 123.82125) (end 83.34 130.13) (width 0.2) (layer "F.Cu") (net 13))
 (segment (start 79.68225 117.9615) (end 78.58125 119.0625) (width 0.2) (layer "F.Cu") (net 13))
 (segment (start 78.58125 107.15625) (end 79.68225 108.25725) (width 0.2) (layer "F.Cu") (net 13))
 (segment (start 96.274 130.81975) (end 97 130.09375) (width 0.2) (layer "F.Cu") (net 13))
 (segment (start 84.02975 130.81975) (end 96.274 130.81975) (width 0.2) (layer "F.Cu") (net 13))
 (segment (start 114.45875 85.56625) (end 114.3 85.725) (width 0.2) (layer "F.Cu") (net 13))
 (segment (start 107.03097 130.09375) (end 113.61722 123.5075) (width 0.2) (layer "F.Cu") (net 13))
 (segment (start 114.45875 104.4575) (end 114.45875 123.5075) (width 0.2) (layer "F.Cu") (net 13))
 (segment (start 97 130.09375) (end 107.03097 130.09375) (width 0.2) (layer "F.Cu") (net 13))
 (segment (start 121.44375 138.1125) (end 100.0125 138.1125) (width 0.2) (layer "F.Cu") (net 6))
 (segment (start 84.61769 94.24) (end 96.25469 82.603) (width 0.2) (layer "F.Cu") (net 6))
 (segment (start 120.703 82.603) (end 121.44375 83.34375) (width 0.2) (layer "F.Cu") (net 6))
 (segment (start 96.25469 82.603) (end 120.703 82.603) (width 0.2) (layer "F.Cu") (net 6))
 (segment (start 81.455 94.24) (end 84.61769 94.24) (width 0.2) (layer "F.Cu") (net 6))
 (segment (start 121.44375 83.34375) (end 121.44375 138.1125) (width 0.2) (layer "F.Cu") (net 6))
 (segment (start 100.0125 138.1125) (end 93.74375 131.84375) (width 0.2) (layer "F.Cu") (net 6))
 (segment (start 93.74375 131.84375) (end 92.86875 131.84375) (width 0.2) (layer "F.Cu") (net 6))
 (segment (start 80.37737 89.16) (end 81.455 89.16) (width 0.2) (layer "F.Cu") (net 4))
 (segment (start 78.58125 120.8125) (end 76.4 118.63125) (width 0.2) (layer "F.Cu") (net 4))
 (segment (start 76.4 118.63125) (end 76.4 93.13737) (width 0.2) (layer "F.Cu") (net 4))
 (segment (start 76.4 93.13737) (end 80.37737 89.16) (width 0.2) (layer "F.Cu") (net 4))
 (segment (start 76.801 109.5375) (end 77.95 109.5375) (width 0.2) (layer "F.Cu") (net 7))
 (segment (start 76.801 100.599) (end 76.801 109.5375) (width 0.2) (layer "F.Cu") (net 7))
 (segment (start 80.62 96.78) (end 76.801 100.599) (width 0.2) (layer "F.Cu") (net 7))
 (segment (start 77.95 109.5375) (end 78.58125 108.90625) (width 0.2) (layer "F.Cu") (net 7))
 (segment (start 89.05875 111.76) (end 96.695 104.12375) (width 0.2) (layer "F.Cu") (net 8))
 (segment (start 96.695 104.12375) (end 96.695 96.78) (width 0.2) (layer "F.Cu") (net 8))
 (segment (start 108.10875 122.740686) (end 95.989064 110.621) (width 0.2) (layer "F.Cu") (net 9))
 (segment (start 108.10875 126.0475) (end 108.10875 122.740686) (width 0.2) (layer "F.Cu") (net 9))
 (segment (start 99.047 95.757) (end 97.53 94.24) (width 0.2) (layer "F.Cu") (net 9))
 (segment (start 94.00775 109.800314) (end 94.00775 107.3781) (width 0.2) (layer "F.Cu") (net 9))
 (segment (start 99.047 102.33885) (end 99.047 95.757) (width 0.2) (layer "F.Cu") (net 9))
 (segment (start 94.00775 107.3781) (end 99.047 102.33885) (width 0.2) (layer "F.Cu") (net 9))
 (segment (start 94.828436 110.621) (end 94.00775 109.800314) (width 0.2) (layer "F.Cu") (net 9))
 (segment (start 95.989064 110.621) (end 94.828436 110.621) (width 0.2) (layer "F.Cu") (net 9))
 (segment (start 86.58775 99.26725) (end 96.695 89.16) (width 0.2) (layer "F.Cu") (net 11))
 (segment (start 108.10875 106.9975) (end 109.50975 108.3985) (width 0.2) (layer "F.Cu") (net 11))
 (segment (start 88.44128 116.651) (end 86.58775 114.79747) (width 0.2) (layer "F.Cu") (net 11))
 (segment (start 86.58775 114.79747) (end 86.58775 99.26725) (width 0.2) (layer "F.Cu") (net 11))
 (segment (start 107.463328 127.513608) (end 96.60072 116.651) (width 0.2) (layer "F.Cu") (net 11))
 (segment (start 109.50975 126.627814) (end 108.623956 127.513608) (width 0.2) (layer "F.Cu") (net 11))
 (segment (start 108.623956 127.513608) (end 107.463328 127.513608) (width 0.2) (layer "F.Cu") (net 11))
 (segment (start 96.60072 116.651) (end 88.44128 116.651) (width 0.2) (layer "F.Cu") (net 11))
 (segment (start 109.50975 108.3985) (end 109.50975 126.627814) (width 0.2) (layer "F.Cu") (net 11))
 (segment (start 108.10875 87.9475) (end 106.553116 87.9475) (width 0.2) (layer "F.Cu") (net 10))
 (segment (start 102.800616 91.7) (end 96.695 91.7) (width 0.2) (layer "F.Cu") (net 10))
 (segment (start 106.553116 87.9475) (end 102.800616 91.7) (width 0.2) (layer "F.Cu") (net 10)))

